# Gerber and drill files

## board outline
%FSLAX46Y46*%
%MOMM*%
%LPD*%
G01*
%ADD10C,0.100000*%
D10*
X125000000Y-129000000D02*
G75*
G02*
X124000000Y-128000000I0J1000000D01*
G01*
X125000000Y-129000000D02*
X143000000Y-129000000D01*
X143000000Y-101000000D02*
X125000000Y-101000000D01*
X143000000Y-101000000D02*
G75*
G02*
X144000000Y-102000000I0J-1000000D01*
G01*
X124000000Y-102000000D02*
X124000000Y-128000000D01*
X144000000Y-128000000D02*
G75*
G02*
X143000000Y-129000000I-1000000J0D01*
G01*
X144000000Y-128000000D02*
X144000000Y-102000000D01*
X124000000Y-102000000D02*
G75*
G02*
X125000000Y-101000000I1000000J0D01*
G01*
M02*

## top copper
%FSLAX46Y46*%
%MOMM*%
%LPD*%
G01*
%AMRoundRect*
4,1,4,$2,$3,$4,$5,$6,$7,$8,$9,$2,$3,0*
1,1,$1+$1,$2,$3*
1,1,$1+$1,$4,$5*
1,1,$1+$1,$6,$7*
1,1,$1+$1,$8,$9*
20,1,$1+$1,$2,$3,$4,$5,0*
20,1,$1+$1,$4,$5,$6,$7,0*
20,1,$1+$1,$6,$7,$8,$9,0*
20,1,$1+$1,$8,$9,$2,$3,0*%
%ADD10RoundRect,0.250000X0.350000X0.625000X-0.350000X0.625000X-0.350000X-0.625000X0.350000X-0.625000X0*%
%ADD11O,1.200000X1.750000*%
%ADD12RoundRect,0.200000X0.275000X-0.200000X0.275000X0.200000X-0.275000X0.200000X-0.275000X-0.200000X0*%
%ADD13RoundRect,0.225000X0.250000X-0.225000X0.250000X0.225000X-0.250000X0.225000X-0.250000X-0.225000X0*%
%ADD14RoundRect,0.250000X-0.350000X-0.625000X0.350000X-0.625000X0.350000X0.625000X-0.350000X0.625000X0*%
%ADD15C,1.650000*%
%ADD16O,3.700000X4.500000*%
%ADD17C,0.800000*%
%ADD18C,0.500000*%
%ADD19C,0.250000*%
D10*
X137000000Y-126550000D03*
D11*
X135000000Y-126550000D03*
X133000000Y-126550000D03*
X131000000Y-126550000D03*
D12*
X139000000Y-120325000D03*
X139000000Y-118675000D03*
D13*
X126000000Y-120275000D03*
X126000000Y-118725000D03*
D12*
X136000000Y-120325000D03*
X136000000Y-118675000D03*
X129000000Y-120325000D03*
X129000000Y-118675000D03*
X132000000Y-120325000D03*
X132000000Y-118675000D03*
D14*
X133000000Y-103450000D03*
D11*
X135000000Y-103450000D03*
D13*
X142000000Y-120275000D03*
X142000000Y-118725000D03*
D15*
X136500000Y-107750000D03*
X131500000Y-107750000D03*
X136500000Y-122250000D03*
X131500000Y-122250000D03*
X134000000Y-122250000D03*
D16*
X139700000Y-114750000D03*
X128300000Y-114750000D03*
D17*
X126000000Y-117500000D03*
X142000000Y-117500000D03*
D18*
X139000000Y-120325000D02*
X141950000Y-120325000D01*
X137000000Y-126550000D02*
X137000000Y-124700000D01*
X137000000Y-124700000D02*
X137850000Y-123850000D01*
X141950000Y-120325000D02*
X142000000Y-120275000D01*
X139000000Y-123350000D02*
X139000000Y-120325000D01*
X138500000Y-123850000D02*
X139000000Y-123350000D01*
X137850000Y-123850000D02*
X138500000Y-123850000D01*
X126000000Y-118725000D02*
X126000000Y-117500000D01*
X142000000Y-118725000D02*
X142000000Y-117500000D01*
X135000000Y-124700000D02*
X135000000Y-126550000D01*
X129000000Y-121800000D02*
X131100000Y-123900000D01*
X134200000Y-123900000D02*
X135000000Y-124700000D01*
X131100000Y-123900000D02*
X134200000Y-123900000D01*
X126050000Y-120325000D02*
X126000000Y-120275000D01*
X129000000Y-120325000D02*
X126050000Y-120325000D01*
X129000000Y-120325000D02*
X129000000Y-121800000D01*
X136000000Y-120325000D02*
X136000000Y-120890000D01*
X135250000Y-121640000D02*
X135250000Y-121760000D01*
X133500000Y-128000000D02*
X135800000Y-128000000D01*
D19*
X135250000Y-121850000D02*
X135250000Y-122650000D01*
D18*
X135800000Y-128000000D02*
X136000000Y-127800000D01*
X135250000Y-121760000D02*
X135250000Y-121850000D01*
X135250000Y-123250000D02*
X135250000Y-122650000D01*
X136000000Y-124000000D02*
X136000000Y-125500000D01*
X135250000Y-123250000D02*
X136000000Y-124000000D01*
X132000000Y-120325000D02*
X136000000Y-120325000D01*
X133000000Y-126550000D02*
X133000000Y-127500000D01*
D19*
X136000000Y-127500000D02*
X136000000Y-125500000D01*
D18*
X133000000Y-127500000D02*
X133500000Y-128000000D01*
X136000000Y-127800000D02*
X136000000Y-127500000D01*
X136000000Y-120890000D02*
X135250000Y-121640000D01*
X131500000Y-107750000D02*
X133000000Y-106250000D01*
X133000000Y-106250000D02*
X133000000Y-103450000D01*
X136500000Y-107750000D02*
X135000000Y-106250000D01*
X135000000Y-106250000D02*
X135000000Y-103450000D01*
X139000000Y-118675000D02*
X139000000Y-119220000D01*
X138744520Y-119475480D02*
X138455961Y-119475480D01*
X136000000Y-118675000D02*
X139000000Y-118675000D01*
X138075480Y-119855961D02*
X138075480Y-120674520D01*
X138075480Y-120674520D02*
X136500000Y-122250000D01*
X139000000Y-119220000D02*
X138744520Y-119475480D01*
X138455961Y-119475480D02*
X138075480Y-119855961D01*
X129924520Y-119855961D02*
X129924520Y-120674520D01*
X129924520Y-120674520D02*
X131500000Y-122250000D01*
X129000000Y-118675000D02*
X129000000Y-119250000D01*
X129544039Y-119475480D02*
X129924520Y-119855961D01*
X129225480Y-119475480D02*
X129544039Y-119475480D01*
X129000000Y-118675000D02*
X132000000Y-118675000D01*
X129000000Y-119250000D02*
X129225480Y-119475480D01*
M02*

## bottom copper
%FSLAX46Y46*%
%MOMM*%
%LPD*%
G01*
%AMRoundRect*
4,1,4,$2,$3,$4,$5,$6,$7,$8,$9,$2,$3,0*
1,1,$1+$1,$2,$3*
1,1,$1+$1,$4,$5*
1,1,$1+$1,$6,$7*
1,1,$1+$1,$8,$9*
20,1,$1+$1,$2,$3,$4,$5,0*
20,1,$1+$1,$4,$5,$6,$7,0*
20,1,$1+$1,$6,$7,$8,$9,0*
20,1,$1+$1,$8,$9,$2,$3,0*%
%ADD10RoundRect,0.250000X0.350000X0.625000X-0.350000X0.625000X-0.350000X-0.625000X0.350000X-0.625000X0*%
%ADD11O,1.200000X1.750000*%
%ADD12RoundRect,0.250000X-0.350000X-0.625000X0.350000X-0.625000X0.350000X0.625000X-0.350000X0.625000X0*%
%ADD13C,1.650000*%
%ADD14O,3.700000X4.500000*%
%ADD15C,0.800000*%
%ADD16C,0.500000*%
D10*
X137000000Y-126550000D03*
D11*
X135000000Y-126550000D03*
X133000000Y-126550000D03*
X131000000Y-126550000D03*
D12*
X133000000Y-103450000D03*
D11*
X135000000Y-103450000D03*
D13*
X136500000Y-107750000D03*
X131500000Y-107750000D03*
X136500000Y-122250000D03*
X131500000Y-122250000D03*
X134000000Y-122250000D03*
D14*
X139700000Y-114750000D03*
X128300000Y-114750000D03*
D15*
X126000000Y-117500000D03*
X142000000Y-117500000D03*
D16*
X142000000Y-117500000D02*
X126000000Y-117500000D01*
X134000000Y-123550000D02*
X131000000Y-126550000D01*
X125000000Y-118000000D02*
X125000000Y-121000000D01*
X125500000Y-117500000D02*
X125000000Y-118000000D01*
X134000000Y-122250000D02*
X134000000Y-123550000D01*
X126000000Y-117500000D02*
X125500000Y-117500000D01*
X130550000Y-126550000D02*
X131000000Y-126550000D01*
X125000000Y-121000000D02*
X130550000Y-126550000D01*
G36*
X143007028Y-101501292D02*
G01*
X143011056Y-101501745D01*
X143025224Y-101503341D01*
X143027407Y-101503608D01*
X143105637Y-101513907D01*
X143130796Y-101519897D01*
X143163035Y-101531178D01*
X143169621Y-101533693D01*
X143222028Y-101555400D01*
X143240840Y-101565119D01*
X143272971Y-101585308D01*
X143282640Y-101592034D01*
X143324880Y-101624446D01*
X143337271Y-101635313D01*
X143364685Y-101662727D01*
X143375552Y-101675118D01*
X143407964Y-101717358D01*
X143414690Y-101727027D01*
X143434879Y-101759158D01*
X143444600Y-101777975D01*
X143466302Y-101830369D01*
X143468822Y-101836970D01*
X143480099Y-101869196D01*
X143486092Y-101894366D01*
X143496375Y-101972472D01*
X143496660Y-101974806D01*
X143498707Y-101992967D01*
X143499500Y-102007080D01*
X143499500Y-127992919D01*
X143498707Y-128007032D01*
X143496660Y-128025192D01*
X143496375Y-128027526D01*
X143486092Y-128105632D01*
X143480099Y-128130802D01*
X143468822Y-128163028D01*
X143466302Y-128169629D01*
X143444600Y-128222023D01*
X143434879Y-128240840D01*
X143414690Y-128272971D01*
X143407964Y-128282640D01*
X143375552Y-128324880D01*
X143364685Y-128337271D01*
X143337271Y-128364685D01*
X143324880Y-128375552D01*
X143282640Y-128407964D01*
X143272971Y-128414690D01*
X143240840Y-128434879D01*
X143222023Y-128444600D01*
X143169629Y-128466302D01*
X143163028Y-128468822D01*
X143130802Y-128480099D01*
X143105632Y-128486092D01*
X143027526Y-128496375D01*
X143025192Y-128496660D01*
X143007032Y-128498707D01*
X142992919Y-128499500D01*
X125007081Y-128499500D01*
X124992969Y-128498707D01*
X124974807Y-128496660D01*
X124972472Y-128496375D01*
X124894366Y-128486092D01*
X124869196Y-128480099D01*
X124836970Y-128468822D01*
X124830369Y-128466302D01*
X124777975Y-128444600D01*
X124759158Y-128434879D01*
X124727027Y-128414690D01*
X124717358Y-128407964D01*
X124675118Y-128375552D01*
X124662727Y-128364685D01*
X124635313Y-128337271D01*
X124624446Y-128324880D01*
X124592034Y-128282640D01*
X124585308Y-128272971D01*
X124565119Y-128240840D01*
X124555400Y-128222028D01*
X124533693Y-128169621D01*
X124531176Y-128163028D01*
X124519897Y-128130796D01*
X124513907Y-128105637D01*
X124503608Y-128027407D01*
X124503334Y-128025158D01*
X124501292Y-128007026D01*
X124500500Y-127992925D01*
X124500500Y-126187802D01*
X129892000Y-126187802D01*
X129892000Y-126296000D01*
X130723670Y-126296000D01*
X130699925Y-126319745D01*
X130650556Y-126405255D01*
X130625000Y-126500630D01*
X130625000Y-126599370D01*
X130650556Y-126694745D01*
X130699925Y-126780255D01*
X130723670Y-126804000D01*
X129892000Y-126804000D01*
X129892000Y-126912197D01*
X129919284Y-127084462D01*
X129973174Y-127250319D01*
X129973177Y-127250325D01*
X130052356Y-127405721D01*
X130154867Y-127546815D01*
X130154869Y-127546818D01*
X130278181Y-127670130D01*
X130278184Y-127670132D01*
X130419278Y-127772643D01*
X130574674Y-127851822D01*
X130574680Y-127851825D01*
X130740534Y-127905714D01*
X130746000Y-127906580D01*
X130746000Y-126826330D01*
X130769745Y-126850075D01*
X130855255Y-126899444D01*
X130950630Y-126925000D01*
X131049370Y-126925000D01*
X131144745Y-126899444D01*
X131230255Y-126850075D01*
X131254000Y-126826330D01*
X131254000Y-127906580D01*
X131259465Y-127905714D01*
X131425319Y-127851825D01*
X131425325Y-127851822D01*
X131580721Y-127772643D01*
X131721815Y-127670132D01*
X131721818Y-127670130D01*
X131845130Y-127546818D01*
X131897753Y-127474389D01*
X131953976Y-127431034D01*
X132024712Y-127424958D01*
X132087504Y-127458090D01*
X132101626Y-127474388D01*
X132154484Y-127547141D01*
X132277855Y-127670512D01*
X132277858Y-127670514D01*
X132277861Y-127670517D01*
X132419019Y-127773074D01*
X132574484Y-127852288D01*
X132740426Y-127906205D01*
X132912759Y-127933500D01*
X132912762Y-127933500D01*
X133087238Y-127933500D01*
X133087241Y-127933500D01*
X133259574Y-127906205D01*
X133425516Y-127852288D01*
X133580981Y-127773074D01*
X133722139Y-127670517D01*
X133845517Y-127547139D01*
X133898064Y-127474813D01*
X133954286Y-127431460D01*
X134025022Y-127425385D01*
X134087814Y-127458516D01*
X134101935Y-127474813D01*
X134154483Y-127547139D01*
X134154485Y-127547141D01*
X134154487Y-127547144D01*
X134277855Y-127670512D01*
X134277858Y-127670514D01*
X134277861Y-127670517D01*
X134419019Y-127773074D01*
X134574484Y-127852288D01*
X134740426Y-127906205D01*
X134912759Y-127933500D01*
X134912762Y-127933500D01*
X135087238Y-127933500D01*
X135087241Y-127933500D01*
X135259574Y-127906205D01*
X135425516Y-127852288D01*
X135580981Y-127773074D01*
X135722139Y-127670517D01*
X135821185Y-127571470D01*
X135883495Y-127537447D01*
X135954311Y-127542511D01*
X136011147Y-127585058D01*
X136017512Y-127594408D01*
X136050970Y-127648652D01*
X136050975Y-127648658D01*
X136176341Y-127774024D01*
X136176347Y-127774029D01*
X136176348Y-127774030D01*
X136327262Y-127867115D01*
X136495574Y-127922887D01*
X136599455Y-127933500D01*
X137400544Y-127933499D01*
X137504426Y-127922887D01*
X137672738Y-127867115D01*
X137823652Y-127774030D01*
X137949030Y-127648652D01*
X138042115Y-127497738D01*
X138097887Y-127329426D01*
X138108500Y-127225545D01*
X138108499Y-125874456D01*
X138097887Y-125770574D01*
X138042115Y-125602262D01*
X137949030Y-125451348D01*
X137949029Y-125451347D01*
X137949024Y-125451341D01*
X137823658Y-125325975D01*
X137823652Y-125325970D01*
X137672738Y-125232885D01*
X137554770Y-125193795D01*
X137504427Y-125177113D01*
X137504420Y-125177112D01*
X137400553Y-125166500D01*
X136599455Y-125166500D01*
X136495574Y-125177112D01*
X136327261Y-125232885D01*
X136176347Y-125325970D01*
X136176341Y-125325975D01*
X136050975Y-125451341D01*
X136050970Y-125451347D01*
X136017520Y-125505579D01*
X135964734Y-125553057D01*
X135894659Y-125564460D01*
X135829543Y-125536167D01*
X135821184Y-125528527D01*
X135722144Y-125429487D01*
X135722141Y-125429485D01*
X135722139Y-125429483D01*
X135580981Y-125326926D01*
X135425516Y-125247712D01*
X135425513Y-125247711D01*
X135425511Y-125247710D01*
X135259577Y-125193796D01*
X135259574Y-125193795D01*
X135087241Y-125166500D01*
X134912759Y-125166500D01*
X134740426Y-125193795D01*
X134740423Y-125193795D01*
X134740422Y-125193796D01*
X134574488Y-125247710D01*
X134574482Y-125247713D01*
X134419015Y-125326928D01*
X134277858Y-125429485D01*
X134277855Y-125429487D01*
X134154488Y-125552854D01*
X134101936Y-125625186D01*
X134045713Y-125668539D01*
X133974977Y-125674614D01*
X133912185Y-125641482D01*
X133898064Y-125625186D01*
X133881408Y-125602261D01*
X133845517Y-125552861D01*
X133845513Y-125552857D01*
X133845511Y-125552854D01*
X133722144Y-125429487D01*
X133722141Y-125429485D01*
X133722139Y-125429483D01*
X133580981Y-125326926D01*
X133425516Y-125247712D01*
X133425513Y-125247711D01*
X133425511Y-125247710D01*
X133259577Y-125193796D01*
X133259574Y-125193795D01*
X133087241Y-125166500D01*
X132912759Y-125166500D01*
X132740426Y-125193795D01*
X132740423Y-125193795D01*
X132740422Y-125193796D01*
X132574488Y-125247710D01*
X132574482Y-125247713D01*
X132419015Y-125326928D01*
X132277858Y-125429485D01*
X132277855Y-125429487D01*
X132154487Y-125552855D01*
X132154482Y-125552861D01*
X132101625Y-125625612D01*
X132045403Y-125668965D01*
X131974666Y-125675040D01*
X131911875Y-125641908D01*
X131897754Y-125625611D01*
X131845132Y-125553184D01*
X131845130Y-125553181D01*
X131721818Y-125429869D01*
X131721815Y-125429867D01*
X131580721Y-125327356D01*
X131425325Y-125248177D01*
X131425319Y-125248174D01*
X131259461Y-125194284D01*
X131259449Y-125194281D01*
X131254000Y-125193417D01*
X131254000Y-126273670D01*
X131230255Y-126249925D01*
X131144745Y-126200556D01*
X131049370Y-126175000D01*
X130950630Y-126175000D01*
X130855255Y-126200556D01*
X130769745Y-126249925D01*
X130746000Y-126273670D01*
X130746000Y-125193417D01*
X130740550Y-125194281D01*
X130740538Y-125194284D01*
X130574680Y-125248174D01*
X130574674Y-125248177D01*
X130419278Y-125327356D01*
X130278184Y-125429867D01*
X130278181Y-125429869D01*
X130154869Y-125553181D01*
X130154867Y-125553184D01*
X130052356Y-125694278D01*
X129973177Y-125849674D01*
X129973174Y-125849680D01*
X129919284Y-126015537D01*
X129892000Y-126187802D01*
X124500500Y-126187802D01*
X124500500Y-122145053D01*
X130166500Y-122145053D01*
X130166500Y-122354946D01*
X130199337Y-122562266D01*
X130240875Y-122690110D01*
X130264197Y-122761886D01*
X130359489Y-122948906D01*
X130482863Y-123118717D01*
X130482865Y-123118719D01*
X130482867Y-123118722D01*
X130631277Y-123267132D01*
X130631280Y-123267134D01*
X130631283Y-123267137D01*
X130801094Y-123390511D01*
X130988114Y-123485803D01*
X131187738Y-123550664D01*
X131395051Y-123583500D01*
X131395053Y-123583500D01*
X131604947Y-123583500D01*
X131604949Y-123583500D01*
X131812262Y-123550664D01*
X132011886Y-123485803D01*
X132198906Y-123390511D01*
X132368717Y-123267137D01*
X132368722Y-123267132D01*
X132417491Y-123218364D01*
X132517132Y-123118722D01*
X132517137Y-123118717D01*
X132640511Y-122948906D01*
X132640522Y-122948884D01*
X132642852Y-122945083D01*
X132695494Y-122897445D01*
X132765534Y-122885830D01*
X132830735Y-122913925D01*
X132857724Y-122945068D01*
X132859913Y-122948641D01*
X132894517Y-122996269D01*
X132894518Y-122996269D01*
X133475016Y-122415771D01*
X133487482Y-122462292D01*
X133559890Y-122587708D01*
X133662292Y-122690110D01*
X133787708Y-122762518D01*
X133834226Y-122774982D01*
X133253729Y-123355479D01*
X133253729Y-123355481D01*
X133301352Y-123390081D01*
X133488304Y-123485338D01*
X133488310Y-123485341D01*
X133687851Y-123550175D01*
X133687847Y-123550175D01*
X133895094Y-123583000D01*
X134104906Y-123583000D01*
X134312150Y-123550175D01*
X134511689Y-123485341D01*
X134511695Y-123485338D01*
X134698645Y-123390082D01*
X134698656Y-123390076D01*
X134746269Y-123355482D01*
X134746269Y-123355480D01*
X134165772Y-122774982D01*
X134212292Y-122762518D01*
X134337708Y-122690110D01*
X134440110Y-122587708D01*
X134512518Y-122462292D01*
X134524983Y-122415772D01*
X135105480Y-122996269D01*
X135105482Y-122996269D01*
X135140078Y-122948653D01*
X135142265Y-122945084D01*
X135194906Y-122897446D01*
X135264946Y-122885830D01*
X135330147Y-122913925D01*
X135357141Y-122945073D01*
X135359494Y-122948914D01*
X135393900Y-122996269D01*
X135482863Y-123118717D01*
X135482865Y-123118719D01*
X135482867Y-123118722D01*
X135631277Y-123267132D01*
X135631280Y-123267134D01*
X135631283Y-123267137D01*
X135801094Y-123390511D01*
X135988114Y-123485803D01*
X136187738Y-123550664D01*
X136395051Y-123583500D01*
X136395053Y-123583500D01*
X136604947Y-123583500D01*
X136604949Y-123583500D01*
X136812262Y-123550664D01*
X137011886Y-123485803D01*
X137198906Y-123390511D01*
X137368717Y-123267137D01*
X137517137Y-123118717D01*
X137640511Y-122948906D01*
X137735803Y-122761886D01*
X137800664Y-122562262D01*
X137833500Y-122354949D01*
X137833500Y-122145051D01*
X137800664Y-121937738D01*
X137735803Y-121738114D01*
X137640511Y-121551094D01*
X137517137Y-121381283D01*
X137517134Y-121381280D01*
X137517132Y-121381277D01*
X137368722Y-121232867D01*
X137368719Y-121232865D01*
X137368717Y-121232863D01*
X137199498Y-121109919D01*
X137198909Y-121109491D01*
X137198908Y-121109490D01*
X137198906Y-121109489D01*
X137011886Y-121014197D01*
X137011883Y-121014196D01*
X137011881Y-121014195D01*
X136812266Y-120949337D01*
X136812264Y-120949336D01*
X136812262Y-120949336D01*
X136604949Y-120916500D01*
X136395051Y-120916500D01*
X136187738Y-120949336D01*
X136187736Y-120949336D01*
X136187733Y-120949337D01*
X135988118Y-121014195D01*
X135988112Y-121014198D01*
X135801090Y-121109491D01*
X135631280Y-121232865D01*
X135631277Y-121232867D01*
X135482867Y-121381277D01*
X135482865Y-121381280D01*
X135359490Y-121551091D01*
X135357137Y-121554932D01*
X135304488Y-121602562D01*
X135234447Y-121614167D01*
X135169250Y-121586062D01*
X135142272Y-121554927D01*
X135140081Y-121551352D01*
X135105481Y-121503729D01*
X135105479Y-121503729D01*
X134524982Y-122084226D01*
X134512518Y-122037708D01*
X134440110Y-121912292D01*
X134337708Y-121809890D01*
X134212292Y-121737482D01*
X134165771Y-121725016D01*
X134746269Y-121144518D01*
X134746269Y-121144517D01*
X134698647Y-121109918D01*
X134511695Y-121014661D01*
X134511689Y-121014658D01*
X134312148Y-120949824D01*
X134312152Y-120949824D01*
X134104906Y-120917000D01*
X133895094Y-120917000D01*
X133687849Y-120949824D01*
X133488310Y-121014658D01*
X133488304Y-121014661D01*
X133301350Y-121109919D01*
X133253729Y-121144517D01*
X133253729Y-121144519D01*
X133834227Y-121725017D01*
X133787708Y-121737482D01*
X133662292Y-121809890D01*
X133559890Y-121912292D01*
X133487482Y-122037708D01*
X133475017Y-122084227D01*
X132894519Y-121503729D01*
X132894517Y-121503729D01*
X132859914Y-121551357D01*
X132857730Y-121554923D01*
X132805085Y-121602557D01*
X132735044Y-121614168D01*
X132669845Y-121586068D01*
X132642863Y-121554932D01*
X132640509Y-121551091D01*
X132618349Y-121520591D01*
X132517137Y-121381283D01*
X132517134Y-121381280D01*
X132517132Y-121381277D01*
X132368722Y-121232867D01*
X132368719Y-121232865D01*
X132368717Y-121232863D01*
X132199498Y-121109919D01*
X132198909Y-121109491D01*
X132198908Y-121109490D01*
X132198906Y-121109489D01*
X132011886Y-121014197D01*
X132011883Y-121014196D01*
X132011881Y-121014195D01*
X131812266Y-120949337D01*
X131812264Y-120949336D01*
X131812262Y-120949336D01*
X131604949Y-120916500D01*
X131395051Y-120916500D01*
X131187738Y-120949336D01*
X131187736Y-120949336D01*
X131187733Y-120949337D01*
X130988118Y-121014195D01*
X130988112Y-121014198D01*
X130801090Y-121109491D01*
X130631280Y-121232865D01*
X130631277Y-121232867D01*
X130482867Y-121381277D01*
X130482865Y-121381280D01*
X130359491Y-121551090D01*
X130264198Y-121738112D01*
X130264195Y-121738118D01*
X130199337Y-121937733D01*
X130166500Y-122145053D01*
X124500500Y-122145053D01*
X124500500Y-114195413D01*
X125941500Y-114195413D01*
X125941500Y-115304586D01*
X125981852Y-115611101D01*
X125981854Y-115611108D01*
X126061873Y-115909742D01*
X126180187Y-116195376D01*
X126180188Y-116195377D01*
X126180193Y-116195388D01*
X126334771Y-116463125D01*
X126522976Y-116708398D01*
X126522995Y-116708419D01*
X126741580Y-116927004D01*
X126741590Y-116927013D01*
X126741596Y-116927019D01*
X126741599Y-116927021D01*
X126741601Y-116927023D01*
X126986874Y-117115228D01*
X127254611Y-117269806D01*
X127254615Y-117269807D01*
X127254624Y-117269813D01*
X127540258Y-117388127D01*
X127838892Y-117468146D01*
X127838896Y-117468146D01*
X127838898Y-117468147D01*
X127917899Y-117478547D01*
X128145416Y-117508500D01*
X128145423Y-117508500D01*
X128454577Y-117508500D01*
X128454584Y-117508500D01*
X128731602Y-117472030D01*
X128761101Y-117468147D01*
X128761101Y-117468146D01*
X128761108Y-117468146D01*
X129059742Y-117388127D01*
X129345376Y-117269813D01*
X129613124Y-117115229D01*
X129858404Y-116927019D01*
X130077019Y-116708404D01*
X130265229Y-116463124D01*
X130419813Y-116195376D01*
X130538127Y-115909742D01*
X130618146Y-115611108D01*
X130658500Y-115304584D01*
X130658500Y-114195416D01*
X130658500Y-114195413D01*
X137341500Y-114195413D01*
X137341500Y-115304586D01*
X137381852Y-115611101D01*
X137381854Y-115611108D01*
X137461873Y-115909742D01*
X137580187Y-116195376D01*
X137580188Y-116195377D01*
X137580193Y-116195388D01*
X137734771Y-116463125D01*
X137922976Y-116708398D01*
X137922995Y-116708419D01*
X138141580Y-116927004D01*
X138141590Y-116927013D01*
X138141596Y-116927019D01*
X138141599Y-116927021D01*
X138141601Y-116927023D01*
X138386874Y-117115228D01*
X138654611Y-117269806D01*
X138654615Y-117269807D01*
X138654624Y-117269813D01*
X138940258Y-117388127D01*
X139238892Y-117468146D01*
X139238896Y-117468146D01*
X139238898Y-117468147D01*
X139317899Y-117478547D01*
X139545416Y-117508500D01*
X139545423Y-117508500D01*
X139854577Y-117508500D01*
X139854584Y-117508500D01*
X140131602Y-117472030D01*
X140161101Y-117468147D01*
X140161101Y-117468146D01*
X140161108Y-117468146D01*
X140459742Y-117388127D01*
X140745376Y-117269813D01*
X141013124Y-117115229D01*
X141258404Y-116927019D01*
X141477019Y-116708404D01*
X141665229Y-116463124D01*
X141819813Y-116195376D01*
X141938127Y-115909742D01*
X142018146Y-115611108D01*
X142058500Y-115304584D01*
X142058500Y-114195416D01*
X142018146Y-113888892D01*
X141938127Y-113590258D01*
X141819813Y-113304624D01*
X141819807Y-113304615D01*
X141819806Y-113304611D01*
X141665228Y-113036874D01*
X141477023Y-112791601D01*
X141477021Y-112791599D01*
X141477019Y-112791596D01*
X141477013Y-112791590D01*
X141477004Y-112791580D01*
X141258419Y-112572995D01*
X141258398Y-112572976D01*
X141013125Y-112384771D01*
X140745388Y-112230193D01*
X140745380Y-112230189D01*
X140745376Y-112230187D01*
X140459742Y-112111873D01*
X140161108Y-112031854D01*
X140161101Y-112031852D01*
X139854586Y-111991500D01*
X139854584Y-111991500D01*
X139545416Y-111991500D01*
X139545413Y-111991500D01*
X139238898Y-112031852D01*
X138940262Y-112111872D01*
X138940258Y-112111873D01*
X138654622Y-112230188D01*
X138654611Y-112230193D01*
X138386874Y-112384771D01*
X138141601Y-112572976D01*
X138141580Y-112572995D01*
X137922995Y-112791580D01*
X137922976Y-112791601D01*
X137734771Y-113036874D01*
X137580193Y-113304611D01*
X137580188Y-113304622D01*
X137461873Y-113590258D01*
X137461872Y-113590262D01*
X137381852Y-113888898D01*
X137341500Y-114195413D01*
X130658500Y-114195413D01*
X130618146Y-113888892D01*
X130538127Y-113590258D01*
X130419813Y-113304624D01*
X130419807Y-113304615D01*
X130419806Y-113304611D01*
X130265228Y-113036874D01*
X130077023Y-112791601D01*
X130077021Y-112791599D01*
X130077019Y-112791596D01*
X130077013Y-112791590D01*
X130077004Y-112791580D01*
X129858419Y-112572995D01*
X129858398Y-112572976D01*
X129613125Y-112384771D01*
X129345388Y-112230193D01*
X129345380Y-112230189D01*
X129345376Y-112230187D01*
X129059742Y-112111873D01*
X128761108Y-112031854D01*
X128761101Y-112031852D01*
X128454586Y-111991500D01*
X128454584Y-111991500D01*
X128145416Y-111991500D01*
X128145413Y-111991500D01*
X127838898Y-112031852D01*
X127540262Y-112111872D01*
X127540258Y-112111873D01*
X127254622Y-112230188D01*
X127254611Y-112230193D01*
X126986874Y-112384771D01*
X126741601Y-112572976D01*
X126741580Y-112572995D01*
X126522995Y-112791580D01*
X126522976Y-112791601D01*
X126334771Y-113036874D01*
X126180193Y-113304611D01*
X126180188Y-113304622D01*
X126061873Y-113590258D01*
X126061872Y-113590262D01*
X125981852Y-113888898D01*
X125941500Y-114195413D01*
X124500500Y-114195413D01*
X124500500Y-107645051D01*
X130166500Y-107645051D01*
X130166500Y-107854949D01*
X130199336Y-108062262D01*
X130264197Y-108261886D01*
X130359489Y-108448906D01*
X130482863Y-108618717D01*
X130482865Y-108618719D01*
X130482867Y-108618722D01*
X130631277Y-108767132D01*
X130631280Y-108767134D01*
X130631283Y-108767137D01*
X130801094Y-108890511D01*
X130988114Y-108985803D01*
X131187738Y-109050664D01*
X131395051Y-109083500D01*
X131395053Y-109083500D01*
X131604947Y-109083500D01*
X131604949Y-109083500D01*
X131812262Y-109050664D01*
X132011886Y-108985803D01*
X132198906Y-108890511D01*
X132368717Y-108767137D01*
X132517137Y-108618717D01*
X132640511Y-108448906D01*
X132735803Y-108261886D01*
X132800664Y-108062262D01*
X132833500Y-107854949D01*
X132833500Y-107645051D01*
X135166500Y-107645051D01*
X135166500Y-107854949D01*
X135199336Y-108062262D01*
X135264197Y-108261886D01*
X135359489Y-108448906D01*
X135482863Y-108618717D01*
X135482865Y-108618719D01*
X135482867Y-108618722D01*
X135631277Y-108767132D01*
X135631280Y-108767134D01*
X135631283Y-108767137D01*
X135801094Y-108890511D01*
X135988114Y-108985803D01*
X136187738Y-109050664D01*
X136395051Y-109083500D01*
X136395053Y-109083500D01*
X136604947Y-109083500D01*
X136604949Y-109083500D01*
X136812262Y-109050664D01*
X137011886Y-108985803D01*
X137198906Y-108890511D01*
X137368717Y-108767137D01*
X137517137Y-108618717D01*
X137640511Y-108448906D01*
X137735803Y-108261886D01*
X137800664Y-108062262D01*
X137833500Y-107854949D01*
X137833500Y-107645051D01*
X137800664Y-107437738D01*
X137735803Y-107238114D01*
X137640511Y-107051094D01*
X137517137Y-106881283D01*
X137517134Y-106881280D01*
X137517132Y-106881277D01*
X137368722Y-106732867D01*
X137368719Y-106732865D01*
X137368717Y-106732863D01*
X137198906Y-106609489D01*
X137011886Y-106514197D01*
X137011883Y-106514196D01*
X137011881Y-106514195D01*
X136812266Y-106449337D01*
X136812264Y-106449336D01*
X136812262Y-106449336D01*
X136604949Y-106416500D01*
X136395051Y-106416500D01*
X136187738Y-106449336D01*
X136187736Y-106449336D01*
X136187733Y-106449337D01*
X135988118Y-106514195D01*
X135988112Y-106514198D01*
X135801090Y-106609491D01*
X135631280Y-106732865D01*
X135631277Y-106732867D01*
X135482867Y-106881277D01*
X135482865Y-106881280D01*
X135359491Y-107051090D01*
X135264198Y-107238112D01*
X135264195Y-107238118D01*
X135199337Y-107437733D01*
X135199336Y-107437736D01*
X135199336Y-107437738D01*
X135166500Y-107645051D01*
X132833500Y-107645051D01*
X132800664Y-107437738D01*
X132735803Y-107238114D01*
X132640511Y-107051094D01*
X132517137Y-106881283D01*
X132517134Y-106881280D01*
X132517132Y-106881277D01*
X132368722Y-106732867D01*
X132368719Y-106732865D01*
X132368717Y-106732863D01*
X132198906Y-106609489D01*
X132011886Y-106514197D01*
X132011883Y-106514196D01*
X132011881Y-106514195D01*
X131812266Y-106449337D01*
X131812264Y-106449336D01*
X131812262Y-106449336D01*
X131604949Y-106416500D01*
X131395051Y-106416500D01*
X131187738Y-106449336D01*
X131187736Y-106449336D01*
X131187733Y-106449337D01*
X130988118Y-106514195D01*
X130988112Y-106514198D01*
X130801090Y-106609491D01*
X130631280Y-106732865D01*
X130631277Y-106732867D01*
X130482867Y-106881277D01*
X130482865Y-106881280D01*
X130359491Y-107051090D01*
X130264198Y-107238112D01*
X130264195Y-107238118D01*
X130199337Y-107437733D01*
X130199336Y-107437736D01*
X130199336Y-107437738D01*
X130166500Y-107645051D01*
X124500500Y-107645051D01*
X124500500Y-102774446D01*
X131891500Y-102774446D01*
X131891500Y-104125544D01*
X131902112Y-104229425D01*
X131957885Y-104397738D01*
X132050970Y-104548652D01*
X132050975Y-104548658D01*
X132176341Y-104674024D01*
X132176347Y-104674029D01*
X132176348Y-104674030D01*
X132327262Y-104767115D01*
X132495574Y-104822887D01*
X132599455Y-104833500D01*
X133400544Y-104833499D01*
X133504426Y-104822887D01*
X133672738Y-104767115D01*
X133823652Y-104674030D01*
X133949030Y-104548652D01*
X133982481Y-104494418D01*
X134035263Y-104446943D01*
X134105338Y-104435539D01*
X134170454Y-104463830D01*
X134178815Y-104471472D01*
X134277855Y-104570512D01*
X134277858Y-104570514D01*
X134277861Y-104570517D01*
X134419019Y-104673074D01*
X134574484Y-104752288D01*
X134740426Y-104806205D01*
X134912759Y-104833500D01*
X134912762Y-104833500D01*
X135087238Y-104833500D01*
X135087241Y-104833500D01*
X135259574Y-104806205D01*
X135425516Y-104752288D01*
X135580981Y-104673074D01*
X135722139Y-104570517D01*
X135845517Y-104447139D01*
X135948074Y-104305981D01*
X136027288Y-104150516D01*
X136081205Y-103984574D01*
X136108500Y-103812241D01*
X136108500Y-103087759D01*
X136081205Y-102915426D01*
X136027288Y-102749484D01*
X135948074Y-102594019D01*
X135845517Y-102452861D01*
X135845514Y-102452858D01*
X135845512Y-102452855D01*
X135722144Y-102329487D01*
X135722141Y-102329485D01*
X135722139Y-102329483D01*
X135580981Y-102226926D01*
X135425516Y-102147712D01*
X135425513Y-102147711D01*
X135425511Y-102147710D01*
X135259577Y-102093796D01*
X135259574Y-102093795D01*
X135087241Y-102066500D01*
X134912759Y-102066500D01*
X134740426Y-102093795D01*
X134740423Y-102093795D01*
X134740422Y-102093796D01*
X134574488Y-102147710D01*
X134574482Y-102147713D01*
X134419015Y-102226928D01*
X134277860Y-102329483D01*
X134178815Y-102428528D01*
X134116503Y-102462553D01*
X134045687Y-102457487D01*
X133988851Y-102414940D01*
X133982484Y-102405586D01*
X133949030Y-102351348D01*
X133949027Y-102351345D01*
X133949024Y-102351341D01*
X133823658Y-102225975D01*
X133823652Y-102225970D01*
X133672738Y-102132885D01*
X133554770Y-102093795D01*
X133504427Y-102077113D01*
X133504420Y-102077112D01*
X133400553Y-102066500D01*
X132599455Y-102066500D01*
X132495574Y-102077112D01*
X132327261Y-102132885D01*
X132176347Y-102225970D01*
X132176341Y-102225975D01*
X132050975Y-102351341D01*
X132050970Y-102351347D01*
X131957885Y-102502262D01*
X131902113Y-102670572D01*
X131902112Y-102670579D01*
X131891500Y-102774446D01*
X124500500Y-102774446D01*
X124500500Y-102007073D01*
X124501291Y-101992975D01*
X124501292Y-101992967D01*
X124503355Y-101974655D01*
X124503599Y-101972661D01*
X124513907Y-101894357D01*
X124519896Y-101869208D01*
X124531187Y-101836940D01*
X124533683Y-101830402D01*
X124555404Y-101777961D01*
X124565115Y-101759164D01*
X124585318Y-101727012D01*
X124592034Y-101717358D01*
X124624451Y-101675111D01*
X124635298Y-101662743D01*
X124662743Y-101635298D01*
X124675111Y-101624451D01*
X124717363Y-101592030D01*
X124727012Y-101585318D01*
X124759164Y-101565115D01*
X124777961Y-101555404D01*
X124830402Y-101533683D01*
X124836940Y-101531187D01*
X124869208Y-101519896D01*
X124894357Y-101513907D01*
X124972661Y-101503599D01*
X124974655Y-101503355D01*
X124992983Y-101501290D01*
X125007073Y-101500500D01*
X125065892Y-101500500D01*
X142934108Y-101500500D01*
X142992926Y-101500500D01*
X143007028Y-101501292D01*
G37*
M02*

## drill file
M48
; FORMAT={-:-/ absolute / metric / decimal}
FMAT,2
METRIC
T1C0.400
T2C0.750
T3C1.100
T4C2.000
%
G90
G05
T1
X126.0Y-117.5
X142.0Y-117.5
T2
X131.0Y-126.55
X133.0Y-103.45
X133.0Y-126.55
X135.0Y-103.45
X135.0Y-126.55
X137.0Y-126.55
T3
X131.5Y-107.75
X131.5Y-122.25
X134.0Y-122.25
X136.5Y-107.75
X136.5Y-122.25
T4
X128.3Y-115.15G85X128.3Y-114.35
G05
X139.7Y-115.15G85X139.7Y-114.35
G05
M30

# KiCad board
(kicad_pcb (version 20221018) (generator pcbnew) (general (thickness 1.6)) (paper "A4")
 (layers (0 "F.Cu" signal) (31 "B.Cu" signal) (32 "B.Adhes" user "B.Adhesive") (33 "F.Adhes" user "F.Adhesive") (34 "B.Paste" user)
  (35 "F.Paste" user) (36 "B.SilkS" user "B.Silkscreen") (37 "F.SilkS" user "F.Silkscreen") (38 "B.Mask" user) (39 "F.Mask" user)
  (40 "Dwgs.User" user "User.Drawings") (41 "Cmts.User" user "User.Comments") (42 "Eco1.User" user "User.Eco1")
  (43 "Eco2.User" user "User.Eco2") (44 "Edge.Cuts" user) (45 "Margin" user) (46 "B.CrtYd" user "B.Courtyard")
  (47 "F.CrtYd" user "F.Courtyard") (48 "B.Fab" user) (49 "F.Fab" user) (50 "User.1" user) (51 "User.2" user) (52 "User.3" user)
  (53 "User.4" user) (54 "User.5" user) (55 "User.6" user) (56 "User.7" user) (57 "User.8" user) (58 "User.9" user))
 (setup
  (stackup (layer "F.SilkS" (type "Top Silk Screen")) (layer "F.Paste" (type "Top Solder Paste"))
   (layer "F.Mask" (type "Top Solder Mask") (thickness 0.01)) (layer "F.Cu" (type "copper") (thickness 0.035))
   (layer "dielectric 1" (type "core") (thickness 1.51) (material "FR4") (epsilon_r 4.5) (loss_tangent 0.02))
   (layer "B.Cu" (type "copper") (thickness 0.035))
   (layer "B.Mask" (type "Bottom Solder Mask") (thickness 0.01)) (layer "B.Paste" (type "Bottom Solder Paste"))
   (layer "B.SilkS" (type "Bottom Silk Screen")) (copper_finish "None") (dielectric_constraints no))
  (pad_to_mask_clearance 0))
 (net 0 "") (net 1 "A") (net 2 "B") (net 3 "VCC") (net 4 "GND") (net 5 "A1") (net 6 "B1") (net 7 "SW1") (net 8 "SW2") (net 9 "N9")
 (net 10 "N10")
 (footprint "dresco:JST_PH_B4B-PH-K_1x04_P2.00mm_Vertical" (layer "F.Cu") (at 137 126.55 180)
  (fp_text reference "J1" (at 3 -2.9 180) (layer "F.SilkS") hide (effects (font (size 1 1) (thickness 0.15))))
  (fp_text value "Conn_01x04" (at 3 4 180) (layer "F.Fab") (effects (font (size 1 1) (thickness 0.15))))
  (pad "1" thru_hole roundrect (at 0 0 180) (size 1.2 1.75) (drill 0.75) (layers "*.Cu" "*.Mask") (roundrect_rratio 0.2083333333)
   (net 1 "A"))
  (pad "2" thru_hole oval (at 2 0 180) (size 1.2 1.75) (drill 0.75) (layers "*.Cu" "*.Mask") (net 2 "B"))
  (pad "3" thru_hole oval (at 4 0 180) (size 1.2 1.75) (drill 0.75) (layers "*.Cu" "*.Mask") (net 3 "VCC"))
  (pad "4" thru_hole oval (at 6 0 180) (size 1.2 1.75) (drill 0.75) (layers "*.Cu" "*.Mask") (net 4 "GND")))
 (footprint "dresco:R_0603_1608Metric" (layer "F.Cu") (at 139 119.5 90)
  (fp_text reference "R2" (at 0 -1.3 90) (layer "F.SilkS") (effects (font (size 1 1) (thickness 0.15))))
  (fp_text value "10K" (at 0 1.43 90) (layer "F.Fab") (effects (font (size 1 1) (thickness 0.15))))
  (pad "1" smd roundrect (at -0.825 0 90) (size 0.8 0.95) (layers "F.Cu" "F.Paste" "F.Mask") (roundrect_rratio 0.25) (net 1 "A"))
  (pad "2" smd roundrect (at 0.825 0 90) (size 0.8 0.95) (layers "F.Cu" "F.Paste" "F.Mask") (roundrect_rratio 0.25) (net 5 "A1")))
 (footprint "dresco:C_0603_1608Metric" (layer "F.Cu") (at 126 119.5 90)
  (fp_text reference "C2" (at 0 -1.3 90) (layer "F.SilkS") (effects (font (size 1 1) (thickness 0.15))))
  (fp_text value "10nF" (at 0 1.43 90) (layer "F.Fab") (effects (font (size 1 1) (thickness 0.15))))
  (pad "1" smd roundrect (at -0.775 0 90) (size 0.9 0.95) (layers "F.Cu" "F.Paste" "F.Mask") (roundrect_rratio 0.25) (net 2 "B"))
  (pad "2" smd roundrect (at 0.775 0 90) (size 0.9 0.95) (layers "F.Cu" "F.Paste" "F.Mask") (roundrect_rratio 0.25) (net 4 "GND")))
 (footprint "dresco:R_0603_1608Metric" (layer "F.Cu") (at 136 119.5 90)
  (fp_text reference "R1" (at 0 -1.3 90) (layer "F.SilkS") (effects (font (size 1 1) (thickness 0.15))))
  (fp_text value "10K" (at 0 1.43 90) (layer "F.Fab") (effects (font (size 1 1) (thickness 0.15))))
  (pad "1" smd roundrect (at -0.825 0 90) (size 0.8 0.95) (layers "F.Cu" "F.Paste" "F.Mask") (roundrect_rratio 0.25) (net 3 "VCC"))
  (pad "2" smd roundrect (at 0.825 0 90) (size 0.8 0.95) (layers "F.Cu" "F.Paste" "F.Mask") (roundrect_rratio 0.25) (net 5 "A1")))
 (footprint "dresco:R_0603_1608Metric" (layer "F.Cu") (at 129 119.5 90)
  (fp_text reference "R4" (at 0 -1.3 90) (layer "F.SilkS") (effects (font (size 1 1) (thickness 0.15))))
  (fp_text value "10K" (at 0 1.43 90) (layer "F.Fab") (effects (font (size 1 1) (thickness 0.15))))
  (pad "1" smd roundrect (at -0.825 0 90) (size 0.8 0.95) (layers "F.Cu" "F.Paste" "F.Mask") (roundrect_rratio 0.25) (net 2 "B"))
  (pad "2" smd roundrect (at 0.825 0 90) (size 0.8 0.95) (layers "F.Cu" "F.Paste" "F.Mask") (roundrect_rratio 0.25) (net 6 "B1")))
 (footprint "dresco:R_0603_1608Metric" (layer "F.Cu") (at 132 119.5 90)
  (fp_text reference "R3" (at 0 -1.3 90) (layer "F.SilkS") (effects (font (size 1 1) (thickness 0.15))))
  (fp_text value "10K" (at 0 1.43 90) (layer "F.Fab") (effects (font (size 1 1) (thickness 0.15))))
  (pad "1" smd roundrect (at -0.825 0 90) (size 0.8 0.95) (layers "F.Cu" "F.Paste" "F.Mask") (roundrect_rratio 0.25) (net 3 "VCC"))
  (pad "2" smd roundrect (at 0.825 0 90) (size 0.8 0.95) (layers "F.Cu" "F.Paste" "F.Mask") (roundrect_rratio 0.25) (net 6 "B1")))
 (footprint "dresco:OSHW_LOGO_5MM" (layer "F.Cu") (at 134 114.5)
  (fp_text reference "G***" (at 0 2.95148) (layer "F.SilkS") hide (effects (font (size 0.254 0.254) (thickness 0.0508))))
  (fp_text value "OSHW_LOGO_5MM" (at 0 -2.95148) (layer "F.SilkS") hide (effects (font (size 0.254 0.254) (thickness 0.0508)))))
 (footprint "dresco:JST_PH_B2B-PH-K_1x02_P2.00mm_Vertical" (layer "F.Cu") (at 133 103.45)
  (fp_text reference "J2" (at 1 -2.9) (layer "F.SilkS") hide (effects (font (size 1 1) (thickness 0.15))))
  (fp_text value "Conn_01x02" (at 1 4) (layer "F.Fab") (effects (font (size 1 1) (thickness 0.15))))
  (pad "1" thru_hole roundrect (at 0 0) (size 1.2 1.75) (drill 0.75) (layers "*.Cu" "*.Mask") (roundrect_rratio 0.2083333333) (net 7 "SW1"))
  (pad "2" thru_hole oval (at 2 0) (size 1.2 1.75) (drill 0.75) (layers "*.Cu" "*.Mask") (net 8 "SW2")))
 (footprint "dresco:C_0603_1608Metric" (layer "F.Cu") (at 142 119.5 90)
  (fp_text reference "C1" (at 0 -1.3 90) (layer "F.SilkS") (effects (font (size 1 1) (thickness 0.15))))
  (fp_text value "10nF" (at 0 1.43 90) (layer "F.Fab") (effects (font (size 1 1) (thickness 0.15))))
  (pad "1" smd roundrect (at -0.775 0 90) (size 0.9 0.95) (layers "F.Cu" "F.Paste" "F.Mask") (roundrect_rratio 0.25) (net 1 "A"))
  (pad "2" smd roundrect (at 0.775 0 90) (size 0.9 0.95) (layers "F.Cu" "F.Paste" "F.Mask") (roundrect_rratio 0.25) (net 4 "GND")))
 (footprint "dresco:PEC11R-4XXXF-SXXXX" (layer "B.Cu") (at 136.5 107.75 180)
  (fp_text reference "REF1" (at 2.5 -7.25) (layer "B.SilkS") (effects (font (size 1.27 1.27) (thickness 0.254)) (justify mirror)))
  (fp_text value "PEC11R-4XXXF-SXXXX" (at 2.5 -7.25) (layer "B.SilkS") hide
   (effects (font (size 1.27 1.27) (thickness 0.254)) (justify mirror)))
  (pad "1" thru_hole circle (at 0 0 180) (size 1.65 1.65) (drill 1.1) (layers "*.Cu" "*.Mask") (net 8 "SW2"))
  (pad "2" thru_hole circle (at 5 0 180) (size 1.65 1.65) (drill 1.1) (layers "*.Cu" "*.Mask") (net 7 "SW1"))
  (pad "A1" thru_hole circle (at 0 -14.5 180) (size 1.65 1.65) (drill 1.1) (layers "*.Cu" "*.Mask") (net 5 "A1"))
  (pad "B1" thru_hole circle (at 5 -14.5 180) (size 1.65 1.65) (drill 1.1) (layers "*.Cu" "*.Mask") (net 6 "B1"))
  (pad "C1" thru_hole circle (at 2.5 -14.5 180) (size 1.65 1.65) (drill 1.1) (layers "*.Cu" "*.Mask") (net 4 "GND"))
  (pad "MH1" thru_hole oval (at -3.2 -7 180) (size 3.7 4.5) (drill oval 2 2.8) (layers "*.Cu" "*.Mask") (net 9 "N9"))
  (pad "MH2" thru_hole oval (at 8.2 -7 180) (size 3.7 4.5) (drill oval 2 2.8) (layers "*.Cu" "*.Mask") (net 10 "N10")))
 (gr_arc (start 125 129) (mid 124.292893 128.707107) (end 124 128) (stroke (width 0.1) (type solid)) (layer "Edge.Cuts"))
 (gr_line (start 125 129) (end 143 129) (stroke (width 0.1) (type solid)) (layer "Edge.Cuts"))
 (gr_line (start 143 101) (end 125 101) (stroke (width 0.1) (type solid)) (layer "Edge.Cuts"))
 (gr_arc (start 143 101) (mid 143.707107 101.292893) (end 144 102) (stroke (width 0.1) (type solid)) (layer "Edge.Cuts"))
 (gr_line (start 124 102) (end 124 128) (stroke (width 0.1) (type solid)) (layer "Edge.Cuts"))
 (gr_arc (start 144 128) (mid 143.707107 128.707107) (end 143 129) (stroke (width 0.1) (type solid)) (layer "Edge.Cuts"))
 (gr_line (start 144 128) (end 144 102) (stroke (width 0.1) (type solid)) (layer "Edge.Cuts"))
 (gr_arc (start 124 102) (mid 124.292893 101.292893) (end 125 101) (stroke (width 0.1) (type solid)) (layer "Edge.Cuts"))
 (segment (start 139 120.325) (end 141.95 120.325) (width 0.5) (layer "F.Cu") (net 1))
 (segment (start 137 126.55) (end 137 124.7) (width 0.5) (layer "F.Cu") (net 1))
 (segment (start 137 124.7) (end 137.85 123.85) (width 0.5) (layer "F.Cu") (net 1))
 (segment (start 141.95 120.325) (end 142 120.275) (width 0.5) (layer "F.Cu") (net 1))
 (segment (start 139 123.35) (end 139 120.325) (width 0.5) (layer "F.Cu") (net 1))
 (segment (start 138.5 123.85) (end 139 123.35) (width 0.5) (layer "F.Cu") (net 1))
 (segment (start 137.85 123.85) (end 138.5 123.85) (width 0.5) (layer "F.Cu") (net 1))
 (segment (start 126 118.725) (end 126 117.5) (width 0.5) (layer "F.Cu") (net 4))
 (segment (start 142 118.725) (end 142 117.5) (width 0.5) (layer "F.Cu") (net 4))
 (via (at 126 117.5) (size 0.8) (drill 0.4) (layers "F.Cu" "B.Cu") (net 4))
 (via (at 142 117.5) (size 0.8) (drill 0.4) (layers "F.Cu" "B.Cu") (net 4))
 (segment (start 142 117.5) (end 126 117.5) (width 0.5) (layer "B.Cu") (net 4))
 (segment (start 134 123.55) (end 131 126.55) (width 0.5) (layer "B.Cu") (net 4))
 (segment (start 125 118) (end 125 121) (width 0.5) (layer "B.Cu") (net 4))
 (segment (start 125.5 117.5) (end 125 118) (width 0.5) (layer "B.Cu") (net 4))
 (segment (start 134 122.25) (end 134 123.55) (width 0.5) (layer "B.Cu") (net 4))
 (segment (start 126 117.5) (end 125.5 117.5) (width 0.5) (layer "B.Cu") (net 4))
 (segment (start 130.55 126.55) (end 131 126.55) (width 0.5) (layer "B.Cu") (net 4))
 (segment (start 125 121) (end 130.55 126.55) (width 0.5) (layer "B.Cu") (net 4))
 (segment (start 135 124.7) (end 135 126.55) (width 0.5) (layer "F.Cu") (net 2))
 (segment (start 129 121.8) (end 131.1 123.9) (width 0.5) (layer "F.Cu") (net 2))
 (segment (start 134.2 123.9) (end 135 124.7) (width 0.5) (layer "F.Cu") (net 2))
 (segment (start 131.1 123.9) (end 134.2 123.9) (width 0.5) (layer "F.Cu") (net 2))
 (segment (start 126.05 120.325) (end 126 120.275) (width 0.5) (layer "F.Cu") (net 2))
 (segment (start 129 120.325) (end 126.05 120.325) (width 0.5) (layer "F.Cu") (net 2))
 (segment (start 129 120.325) (end 129 121.8) (width 0.5) (layer "F.Cu") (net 2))
 (segment (start 136 120.325) (end 136 120.89) (width 0.5) (layer "F.Cu") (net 3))
 (segment (start 135.25 121.64) (end 135.25 121.76) (width 0.5) (layer "F.Cu") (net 3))
 (segment (start 133.5 128) (end 135.8 128) (width 0.5) (layer "F.Cu") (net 3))
 (segment (start 135.25 121.85) (end 135.25 122.65) (width 0.25) (layer "F.Cu") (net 3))
 (segment (start 135.8 128) (end 136 127.8) (width 0.5) (layer "F.Cu") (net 3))
 (segment (start 135.25 121.76) (end 135.25 121.85) (width 0.5) (layer "F.Cu") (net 3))
 (segment (start 135.25 123.25) (end 135.25 122.65) (width 0.5) (layer "F.Cu") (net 3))
 (segment (start 136 124) (end 136 125.5) (width 0.5) (layer "F.Cu") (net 3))
 (segment (start 135.25 123.25) (end 136 124) (width 0.5) (layer "F.Cu") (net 3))
 (segment (start 132 120.325) (end 136 120.325) (width 0.5) (layer "F.Cu") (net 3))
 (segment (start 133 126.55) (end 133 127.5) (width 0.5) (layer "F.Cu") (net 3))
 (segment (start 136 127.5) (end 136 125.5) (width 0.25) (layer "F.Cu") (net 3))
 (segment (start 133 127.5) (end 133.5 128) (width 0.5) (layer "F.Cu") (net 3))
 (segment (start 136 127.8) (end 136 127.5) (width 0.5) (layer "F.Cu") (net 3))
 (segment (start 136 120.89) (end 135.25 121.64) (width 0.5) (layer "F.Cu") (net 3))
 (segment (start 131.5 107.75) (end 133 106.25) (width 0.5) (layer "F.Cu") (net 7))
 (segment (start 133 106.25) (end 133 103.45) (width 0.5) (layer "F.Cu") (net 7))
 (segment (start 136.5 107.75) (end 135 106.25) (width 0.5) (layer "F.Cu") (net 8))
 (segment (start 135 106.25) (end 135 103.45) (width 0.5) (layer "F.Cu") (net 8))
 (segment (start 139 118.675) (end 139 119.22) (width 0.5) (layer "F.Cu") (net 5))
 (segment (start 138.74452 119.47548) (end 138.455961 119.47548) (width 0.5) (layer "F.Cu") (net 5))
 (segment (start 136 118.675) (end 139 118.675) (width 0.5) (layer "F.Cu") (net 5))
 (segment (start 138.07548 119.855961) (end 138.07548 120.67452) (width 0.5) (layer "F.Cu") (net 5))
 (segment (start 138.07548 120.67452) (end 136.5 122.25) (width 0.5) (layer "F.Cu") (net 5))
 (segment (start 139 119.22) (end 138.74452 119.47548) (width 0.5) (layer "F.Cu") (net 5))
 (segment (start 138.455961 119.47548) (end 138.07548 119.855961) (width 0.5) (layer "F.Cu") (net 5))
 (segment (start 129.92452 119.855961) (end 129.92452 120.67452) (width 0.5) (layer "F.Cu") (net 6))
 (segment (start 129.92452 120.67452) (end 131.5 122.25) (width 0.5) (layer "F.Cu") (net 6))
 (segment (start 129 118.675) (end 129 119.25) (width 0.5) (layer "F.Cu") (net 6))
 (segment (start 129.544039 119.47548) (end 129.92452 119.855961) (width 0.5) (layer "F.Cu") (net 6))
 (segment (start 129.22548 119.47548) (end 129.544039 119.47548) (width 0.5) (layer "F.Cu") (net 6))
 (segment (start 129 118.675) (end 132 118.675) (width 0.5) (layer "F.Cu") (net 6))
 (segment (start 129 119.25) (end 129.22548 119.47548) (width 0.5) (layer "F.Cu") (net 6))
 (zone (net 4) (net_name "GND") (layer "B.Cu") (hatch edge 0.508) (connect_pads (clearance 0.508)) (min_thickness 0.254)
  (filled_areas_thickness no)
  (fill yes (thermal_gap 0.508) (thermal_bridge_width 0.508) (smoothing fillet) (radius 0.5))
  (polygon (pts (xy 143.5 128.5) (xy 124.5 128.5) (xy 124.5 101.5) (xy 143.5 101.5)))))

